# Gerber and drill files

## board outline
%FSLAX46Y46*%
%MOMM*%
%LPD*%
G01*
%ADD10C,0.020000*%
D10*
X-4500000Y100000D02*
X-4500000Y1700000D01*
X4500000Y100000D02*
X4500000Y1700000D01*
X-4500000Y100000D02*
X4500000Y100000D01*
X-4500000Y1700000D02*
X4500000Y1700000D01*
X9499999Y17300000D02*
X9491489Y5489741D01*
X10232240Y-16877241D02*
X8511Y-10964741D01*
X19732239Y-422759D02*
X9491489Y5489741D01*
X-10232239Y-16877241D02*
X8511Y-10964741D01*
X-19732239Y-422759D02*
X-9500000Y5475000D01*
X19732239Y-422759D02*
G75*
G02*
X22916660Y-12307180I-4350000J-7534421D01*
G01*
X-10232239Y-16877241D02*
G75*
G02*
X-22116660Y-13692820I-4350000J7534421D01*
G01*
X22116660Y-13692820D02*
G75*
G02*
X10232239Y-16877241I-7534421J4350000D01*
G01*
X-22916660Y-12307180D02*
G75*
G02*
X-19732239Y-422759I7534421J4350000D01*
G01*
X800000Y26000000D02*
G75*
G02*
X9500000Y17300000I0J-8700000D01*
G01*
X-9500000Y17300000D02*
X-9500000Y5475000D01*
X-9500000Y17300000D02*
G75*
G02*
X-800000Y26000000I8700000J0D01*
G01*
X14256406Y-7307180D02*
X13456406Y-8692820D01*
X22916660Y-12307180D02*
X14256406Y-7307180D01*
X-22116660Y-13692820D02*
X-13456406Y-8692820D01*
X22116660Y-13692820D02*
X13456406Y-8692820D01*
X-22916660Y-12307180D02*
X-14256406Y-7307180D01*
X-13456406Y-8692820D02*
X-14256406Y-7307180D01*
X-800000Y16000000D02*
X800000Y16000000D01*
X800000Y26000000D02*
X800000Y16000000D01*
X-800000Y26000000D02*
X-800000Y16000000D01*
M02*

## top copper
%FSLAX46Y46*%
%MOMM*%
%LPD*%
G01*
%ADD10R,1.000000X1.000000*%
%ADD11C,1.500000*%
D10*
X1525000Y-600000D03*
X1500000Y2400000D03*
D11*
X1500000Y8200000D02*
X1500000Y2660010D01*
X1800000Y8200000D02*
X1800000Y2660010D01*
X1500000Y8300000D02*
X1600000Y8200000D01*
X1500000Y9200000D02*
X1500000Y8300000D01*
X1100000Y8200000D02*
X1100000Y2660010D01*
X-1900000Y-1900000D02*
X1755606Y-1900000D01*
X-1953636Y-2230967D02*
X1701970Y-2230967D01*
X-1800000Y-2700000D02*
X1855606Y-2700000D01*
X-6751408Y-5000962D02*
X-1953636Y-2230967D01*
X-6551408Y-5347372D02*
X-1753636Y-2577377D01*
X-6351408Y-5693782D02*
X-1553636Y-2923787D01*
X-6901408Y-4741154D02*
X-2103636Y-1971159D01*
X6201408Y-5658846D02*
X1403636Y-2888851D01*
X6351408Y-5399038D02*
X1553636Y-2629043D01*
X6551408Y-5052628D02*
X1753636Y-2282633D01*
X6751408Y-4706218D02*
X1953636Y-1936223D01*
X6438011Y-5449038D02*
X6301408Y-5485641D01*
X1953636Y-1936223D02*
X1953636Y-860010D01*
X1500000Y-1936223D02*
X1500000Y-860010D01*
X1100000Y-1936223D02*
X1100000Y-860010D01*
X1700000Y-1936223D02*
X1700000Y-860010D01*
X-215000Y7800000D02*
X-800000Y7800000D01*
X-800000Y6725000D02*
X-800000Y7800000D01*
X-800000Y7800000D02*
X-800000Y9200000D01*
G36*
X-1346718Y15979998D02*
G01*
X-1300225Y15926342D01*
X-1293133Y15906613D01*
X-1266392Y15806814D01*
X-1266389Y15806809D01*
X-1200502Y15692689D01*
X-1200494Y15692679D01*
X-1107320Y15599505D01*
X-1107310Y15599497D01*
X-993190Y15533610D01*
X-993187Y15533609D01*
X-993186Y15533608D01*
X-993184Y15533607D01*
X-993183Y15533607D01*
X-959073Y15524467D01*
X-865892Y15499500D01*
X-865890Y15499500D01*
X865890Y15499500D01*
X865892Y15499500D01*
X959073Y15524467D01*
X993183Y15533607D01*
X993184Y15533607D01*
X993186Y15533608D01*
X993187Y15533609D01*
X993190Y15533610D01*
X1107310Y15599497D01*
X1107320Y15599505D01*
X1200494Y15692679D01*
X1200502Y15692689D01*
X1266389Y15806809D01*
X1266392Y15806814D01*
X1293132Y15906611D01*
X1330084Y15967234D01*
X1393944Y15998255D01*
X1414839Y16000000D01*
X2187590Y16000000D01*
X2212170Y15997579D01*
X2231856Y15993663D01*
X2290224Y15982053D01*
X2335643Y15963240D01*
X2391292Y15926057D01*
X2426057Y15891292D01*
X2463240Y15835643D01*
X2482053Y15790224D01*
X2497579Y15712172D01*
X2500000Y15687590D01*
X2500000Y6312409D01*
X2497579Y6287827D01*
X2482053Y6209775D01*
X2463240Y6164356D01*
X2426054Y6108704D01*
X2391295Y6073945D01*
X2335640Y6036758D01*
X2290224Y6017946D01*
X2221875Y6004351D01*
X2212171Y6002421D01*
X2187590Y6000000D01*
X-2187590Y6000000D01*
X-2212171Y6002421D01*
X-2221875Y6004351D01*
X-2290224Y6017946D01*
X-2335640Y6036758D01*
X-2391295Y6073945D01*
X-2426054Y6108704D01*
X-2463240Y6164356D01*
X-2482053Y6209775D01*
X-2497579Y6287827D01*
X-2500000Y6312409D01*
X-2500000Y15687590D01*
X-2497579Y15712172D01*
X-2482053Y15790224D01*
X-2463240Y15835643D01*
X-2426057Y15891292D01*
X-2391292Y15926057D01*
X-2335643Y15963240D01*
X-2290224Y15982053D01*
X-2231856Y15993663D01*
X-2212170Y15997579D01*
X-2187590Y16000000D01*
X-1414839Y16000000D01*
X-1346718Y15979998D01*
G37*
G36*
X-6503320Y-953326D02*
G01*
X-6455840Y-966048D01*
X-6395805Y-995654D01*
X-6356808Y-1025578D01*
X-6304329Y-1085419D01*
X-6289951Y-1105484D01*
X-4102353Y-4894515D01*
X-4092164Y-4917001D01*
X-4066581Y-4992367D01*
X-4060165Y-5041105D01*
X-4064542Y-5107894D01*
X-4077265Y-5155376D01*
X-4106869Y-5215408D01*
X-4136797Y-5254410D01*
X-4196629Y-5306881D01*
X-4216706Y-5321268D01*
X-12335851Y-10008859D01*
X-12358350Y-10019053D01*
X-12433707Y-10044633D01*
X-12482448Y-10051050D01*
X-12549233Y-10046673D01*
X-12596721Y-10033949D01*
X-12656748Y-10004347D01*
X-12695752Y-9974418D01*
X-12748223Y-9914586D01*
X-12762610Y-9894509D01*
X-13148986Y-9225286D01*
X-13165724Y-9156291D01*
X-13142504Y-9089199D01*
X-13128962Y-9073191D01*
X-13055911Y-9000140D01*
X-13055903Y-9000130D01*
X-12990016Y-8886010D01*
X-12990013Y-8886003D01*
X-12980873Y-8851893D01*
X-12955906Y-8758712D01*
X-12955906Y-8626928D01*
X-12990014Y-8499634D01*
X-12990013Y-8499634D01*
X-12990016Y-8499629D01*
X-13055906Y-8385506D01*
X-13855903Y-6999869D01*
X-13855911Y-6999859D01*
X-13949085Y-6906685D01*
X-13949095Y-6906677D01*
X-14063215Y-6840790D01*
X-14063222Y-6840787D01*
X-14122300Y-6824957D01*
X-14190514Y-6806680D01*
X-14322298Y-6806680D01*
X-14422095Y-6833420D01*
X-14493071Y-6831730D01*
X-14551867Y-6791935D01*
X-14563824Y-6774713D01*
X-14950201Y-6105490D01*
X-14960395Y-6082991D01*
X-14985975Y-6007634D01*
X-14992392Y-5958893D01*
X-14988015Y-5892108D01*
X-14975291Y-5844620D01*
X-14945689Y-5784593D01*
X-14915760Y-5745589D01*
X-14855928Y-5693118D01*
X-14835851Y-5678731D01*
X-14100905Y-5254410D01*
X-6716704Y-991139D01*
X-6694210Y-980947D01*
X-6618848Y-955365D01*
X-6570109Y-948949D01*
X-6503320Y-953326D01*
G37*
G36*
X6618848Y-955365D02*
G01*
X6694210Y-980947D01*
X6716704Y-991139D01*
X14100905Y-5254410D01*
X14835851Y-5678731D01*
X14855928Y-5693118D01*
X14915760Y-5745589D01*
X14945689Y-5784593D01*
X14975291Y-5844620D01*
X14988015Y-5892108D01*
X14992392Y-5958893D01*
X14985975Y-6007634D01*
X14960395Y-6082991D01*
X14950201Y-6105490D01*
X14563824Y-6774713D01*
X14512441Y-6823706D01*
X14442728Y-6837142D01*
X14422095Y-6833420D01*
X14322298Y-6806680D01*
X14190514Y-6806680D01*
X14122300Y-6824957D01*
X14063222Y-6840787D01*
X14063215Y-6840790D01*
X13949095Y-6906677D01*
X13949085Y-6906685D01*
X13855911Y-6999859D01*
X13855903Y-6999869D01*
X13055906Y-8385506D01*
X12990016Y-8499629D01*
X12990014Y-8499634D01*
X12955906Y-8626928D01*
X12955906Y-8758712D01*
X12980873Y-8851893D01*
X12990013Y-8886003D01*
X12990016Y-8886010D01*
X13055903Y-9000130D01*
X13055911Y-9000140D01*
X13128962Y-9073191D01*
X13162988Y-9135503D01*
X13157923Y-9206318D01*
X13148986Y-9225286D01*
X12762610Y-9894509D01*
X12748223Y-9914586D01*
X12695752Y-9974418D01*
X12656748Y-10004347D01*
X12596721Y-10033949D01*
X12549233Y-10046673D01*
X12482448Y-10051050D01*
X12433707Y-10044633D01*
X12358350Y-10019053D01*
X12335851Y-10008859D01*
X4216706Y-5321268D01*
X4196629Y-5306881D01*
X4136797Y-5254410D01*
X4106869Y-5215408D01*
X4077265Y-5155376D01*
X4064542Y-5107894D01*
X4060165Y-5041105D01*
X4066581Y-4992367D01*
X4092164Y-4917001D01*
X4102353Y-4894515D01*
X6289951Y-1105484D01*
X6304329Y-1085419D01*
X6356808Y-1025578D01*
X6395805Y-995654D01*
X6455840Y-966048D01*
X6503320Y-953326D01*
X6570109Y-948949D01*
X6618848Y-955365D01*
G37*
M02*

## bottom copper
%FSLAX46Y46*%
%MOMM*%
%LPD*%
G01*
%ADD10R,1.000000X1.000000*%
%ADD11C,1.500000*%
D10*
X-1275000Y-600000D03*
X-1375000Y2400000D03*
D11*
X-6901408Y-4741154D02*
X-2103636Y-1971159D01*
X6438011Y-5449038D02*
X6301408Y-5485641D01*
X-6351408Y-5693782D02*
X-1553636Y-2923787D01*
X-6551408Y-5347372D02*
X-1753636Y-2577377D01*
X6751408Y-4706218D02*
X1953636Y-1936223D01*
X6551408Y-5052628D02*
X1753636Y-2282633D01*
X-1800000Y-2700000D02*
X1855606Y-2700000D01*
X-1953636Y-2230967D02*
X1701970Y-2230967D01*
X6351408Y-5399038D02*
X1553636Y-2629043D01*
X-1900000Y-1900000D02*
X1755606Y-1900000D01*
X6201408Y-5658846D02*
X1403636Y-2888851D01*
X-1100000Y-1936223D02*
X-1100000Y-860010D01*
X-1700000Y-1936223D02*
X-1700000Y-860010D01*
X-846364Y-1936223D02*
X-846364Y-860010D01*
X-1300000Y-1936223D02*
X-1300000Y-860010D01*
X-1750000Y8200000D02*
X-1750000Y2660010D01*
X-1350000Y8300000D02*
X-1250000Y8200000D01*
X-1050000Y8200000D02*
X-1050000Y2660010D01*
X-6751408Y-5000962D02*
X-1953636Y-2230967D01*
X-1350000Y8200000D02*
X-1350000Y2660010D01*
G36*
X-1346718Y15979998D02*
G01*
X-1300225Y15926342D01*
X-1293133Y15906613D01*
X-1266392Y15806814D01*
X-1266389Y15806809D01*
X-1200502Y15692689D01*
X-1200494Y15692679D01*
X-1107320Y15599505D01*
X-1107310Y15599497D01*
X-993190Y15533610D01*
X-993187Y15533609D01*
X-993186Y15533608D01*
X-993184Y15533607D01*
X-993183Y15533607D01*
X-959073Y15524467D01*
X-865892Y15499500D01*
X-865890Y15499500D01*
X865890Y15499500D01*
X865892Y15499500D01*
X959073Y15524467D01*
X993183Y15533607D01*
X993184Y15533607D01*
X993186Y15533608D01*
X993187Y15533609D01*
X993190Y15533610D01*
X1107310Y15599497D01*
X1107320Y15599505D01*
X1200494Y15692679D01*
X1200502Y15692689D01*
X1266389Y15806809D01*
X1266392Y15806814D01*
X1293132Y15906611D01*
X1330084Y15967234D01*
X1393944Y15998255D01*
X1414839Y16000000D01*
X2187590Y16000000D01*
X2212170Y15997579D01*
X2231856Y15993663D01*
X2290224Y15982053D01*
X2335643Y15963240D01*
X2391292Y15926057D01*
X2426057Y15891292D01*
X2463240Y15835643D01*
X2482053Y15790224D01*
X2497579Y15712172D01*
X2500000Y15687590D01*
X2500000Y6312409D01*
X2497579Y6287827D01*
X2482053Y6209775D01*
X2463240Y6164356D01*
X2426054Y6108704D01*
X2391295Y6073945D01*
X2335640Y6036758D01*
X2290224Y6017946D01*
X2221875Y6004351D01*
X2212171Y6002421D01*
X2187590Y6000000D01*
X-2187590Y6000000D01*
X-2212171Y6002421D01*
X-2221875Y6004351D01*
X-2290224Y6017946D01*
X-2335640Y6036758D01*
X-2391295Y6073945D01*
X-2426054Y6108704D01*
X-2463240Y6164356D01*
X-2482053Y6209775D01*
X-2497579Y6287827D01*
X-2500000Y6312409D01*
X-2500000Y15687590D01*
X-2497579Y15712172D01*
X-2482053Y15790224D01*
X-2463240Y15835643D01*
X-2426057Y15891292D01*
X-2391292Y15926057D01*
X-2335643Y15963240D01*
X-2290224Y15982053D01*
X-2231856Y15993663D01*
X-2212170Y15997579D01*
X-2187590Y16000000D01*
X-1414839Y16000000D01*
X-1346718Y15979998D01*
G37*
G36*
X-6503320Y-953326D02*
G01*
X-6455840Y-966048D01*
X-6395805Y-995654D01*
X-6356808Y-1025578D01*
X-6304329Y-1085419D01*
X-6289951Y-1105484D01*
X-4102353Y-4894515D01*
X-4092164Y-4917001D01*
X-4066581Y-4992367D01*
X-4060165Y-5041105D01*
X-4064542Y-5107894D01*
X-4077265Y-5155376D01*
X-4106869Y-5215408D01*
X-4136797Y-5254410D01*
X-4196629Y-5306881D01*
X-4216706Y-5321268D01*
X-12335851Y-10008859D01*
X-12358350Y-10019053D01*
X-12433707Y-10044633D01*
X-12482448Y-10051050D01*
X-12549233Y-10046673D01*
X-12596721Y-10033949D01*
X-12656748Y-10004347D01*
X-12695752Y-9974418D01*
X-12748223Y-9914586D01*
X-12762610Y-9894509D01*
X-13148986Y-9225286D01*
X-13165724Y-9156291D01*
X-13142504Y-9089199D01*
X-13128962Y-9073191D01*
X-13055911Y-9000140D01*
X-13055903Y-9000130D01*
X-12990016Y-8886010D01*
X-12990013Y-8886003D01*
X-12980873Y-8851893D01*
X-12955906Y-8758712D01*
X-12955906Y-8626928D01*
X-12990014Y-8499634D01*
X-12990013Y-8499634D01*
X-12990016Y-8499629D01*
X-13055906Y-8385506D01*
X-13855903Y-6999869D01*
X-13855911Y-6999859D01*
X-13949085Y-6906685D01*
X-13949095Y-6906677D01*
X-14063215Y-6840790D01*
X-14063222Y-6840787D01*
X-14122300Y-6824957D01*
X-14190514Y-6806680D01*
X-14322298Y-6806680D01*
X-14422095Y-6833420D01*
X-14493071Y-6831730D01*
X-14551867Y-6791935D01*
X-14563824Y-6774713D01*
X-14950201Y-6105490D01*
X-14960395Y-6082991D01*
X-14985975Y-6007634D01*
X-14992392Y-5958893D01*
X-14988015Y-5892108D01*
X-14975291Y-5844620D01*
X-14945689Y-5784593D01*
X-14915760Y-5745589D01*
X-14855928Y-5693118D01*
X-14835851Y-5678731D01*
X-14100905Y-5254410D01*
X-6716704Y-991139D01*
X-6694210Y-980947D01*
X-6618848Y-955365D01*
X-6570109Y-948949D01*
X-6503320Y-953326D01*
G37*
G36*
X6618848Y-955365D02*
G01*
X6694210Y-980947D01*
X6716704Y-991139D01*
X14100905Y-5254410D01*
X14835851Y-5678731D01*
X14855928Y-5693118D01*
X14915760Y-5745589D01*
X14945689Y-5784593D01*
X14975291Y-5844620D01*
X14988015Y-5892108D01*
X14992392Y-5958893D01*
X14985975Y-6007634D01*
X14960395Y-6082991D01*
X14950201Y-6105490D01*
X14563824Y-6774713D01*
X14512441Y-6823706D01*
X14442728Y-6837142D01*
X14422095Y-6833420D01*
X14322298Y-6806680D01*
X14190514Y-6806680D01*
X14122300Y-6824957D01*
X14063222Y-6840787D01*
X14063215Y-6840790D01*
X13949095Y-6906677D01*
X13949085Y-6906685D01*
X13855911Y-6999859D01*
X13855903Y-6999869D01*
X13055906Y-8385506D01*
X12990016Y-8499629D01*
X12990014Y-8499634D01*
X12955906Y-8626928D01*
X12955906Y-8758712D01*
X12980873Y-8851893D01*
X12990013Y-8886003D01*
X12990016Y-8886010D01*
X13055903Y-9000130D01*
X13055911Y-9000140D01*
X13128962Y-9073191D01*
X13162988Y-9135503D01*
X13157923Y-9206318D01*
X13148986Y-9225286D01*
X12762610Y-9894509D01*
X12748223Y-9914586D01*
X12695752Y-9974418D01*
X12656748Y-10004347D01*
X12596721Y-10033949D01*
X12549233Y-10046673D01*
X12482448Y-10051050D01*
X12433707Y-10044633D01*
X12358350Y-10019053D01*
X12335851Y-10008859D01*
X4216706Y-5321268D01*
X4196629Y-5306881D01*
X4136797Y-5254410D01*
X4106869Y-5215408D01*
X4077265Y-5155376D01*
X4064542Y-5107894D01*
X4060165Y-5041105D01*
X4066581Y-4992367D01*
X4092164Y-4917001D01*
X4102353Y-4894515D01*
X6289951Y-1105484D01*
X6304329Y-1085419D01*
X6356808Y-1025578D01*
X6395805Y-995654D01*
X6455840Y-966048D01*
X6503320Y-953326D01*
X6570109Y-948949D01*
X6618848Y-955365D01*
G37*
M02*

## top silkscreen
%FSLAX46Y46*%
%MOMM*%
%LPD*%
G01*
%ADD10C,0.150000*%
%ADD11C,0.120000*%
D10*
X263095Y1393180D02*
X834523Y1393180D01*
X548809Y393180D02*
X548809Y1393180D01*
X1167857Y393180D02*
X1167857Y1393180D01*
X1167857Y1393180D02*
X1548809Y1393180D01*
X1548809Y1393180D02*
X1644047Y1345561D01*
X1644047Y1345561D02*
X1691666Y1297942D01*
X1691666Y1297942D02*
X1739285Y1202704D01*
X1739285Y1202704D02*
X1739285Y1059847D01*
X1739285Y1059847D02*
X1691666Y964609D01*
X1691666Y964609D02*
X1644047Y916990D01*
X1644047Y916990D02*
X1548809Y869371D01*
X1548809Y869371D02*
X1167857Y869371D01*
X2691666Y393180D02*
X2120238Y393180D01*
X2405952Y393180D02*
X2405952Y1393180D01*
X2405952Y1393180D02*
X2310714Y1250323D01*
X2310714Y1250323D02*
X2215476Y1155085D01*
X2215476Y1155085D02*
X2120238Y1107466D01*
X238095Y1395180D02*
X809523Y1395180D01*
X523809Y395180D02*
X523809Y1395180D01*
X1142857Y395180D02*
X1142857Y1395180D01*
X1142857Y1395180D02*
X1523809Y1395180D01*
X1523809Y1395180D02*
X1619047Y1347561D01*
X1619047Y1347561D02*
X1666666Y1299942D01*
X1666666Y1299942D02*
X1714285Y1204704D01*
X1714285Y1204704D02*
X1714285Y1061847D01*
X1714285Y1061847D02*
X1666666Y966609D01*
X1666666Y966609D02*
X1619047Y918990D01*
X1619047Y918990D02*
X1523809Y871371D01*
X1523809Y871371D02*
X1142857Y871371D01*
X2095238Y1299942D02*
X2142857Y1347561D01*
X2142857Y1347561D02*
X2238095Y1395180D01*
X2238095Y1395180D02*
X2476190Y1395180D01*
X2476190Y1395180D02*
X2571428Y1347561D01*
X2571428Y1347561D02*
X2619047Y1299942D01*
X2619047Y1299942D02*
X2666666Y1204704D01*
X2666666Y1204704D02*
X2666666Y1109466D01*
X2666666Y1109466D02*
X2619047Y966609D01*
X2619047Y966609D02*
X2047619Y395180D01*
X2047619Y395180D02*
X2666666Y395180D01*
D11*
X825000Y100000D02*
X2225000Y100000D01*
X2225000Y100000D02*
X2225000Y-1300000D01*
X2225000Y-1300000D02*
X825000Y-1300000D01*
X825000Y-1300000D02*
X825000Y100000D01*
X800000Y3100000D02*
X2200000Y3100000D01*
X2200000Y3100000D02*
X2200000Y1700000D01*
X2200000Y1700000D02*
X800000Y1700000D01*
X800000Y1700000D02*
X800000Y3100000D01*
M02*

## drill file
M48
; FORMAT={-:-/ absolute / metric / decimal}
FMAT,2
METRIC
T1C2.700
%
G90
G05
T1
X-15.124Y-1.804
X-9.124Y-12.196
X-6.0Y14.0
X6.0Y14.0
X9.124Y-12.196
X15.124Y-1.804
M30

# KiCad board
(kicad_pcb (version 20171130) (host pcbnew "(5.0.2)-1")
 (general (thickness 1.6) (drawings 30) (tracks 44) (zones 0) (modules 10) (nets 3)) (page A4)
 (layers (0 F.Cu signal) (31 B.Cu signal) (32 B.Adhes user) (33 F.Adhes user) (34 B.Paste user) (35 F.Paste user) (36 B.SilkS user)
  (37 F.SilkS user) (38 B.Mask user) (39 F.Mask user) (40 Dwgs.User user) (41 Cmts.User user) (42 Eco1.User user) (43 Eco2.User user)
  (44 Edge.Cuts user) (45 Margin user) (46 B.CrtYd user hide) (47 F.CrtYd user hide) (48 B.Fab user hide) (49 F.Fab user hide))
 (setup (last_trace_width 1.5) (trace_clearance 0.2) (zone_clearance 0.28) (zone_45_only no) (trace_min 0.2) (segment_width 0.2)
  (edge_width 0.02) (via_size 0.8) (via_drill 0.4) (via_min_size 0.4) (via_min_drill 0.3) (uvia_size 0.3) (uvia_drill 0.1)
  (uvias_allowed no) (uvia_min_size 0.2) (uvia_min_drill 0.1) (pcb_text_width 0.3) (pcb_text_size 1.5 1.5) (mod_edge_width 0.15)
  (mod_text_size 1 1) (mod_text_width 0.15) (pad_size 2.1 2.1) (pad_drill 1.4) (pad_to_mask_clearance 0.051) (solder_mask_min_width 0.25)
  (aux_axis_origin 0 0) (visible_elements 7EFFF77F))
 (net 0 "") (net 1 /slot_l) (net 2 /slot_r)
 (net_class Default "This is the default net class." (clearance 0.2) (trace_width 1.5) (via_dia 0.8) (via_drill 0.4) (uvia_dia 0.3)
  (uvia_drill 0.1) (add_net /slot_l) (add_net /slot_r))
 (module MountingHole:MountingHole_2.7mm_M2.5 (layer F.Cu) (at 15.124356 1.803848 240)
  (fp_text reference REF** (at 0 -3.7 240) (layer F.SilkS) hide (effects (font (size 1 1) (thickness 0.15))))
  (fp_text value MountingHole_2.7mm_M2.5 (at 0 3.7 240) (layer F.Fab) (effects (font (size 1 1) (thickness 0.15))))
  (pad 1 np_thru_hole circle (at 0 0 240) (size 2.7 2.7) (drill 2.7) (layers *.Cu *.Mask)))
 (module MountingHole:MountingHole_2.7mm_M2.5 (layer F.Cu) (at -9.124356 12.196152 120)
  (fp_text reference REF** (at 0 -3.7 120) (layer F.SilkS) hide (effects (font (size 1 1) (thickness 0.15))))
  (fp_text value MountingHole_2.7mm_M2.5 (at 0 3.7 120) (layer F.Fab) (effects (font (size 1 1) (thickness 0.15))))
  (pad 1 np_thru_hole circle (at 0 0 120) (size 2.7 2.7) (drill 2.7) (layers *.Cu *.Mask)))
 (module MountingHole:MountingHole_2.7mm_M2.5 (layer F.Cu) (at 9.124356 12.196152 240)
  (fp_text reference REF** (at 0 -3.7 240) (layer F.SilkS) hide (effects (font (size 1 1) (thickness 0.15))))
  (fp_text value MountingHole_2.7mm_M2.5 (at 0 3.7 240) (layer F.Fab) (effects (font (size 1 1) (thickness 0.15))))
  (pad 1 np_thru_hole circle (at 0 0 240) (size 2.7 2.7) (drill 2.7) (layers *.Cu *.Mask)))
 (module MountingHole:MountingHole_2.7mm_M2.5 (layer F.Cu) (at -15.124356 1.803848 120)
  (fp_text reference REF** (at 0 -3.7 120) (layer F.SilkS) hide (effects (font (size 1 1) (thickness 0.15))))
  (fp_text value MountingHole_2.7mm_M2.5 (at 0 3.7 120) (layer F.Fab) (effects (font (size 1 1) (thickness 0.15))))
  (pad 1 np_thru_hole circle (at 0 0 120) (size 2.7 2.7) (drill 2.7) (layers *.Cu *.Mask)))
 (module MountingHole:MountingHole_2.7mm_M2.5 (layer F.Cu) (at 6 -14)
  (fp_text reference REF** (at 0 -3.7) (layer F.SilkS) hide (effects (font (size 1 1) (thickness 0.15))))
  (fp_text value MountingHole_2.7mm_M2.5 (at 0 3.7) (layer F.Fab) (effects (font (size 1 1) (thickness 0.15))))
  (pad 1 np_thru_hole circle (at 0 0) (size 2.7 2.7) (drill 2.7) (layers *.Cu *.Mask)))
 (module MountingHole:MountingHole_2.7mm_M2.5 (layer F.Cu) (at -6 -14)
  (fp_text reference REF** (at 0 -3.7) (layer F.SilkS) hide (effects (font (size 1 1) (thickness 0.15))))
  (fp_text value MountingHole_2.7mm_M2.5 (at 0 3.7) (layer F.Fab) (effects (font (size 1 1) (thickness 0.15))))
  (pad 1 np_thru_hole circle (at 0 0) (size 2.7 2.7) (drill 2.7) (layers *.Cu *.Mask)))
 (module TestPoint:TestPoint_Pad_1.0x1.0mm (layer F.Cu) (at 1.525 0.6)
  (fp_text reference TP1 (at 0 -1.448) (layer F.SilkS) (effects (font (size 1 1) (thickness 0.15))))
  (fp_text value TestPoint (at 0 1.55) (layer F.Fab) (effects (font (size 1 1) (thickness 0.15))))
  (fp_line (start -0.7 -0.7) (end 0.7 -0.7) (layer F.SilkS) (width 0.12))
  (fp_line (start 0.7 -0.7) (end 0.7 0.7) (layer F.SilkS) (width 0.12))
  (fp_line (start 0.7 0.7) (end -0.7 0.7) (layer F.SilkS) (width 0.12))
  (fp_line (start -0.7 0.7) (end -0.7 -0.7) (layer F.SilkS) (width 0.12))
  (pad 1 smd rect (at 0 0) (size 1 1) (layers F.Cu F.Mask) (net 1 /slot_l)))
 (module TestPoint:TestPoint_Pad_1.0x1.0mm (layer F.Cu) (at 1.5 -2.4)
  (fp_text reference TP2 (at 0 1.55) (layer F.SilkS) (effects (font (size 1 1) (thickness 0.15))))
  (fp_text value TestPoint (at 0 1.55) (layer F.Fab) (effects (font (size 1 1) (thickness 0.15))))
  (fp_line (start -0.7 -0.7) (end 0.7 -0.7) (layer F.SilkS) (width 0.12))
  (fp_line (start 0.7 -0.7) (end 0.7 0.7) (layer F.SilkS) (width 0.12))
  (fp_line (start 0.7 0.7) (end -0.7 0.7) (layer F.SilkS) (width 0.12))
  (fp_line (start -0.7 0.7) (end -0.7 -0.7) (layer F.SilkS) (width 0.12))
  (pad 1 smd rect (at 0 0) (size 1 1) (layers F.Cu F.Mask) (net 1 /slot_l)))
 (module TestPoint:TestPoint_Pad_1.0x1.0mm (layer B.Cu) (at -1.275 0.6)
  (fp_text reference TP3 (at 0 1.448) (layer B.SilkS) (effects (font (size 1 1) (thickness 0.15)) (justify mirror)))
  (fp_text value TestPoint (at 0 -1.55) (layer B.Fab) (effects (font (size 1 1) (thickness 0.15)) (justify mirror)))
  (pad 1 smd rect (at 0 0) (size 1 1) (layers B.Cu B.Mask) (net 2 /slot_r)))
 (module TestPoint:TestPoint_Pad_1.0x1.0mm (layer B.Cu) (at -1.375 -2.4)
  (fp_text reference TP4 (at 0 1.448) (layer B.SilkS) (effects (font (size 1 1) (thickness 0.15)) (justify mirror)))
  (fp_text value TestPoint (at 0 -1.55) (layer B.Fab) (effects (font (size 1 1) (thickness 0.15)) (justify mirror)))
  (pad 1 smd rect (at 0 0) (size 1 1) (layers B.Cu B.Mask) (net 2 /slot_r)))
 (gr_line (start -4.5 -0.1) (end -4.5 -1.7) (layer Edge.Cuts) (width 0.02))
 (gr_line (start 4.5 -0.1) (end 4.5 -1.7) (layer Edge.Cuts) (width 0.02))
 (gr_line (start -4.5 -0.1) (end 4.5 -0.1) (layer Edge.Cuts) (width 0.02))
 (gr_line (start -4.5 -1.7) (end 4.5 -1.7) (layer Edge.Cuts) (width 0.02))
 (gr_line (start 9.499999 -17.3) (end 9.491489 -5.489741) (layer Edge.Cuts) (width 0.02))
 (gr_line (start 10.23224 16.877241) (end 0.008511 10.964741) (layer Edge.Cuts) (width 0.02))
 (gr_line (start 19.732239 0.422759) (end 9.491489 -5.489741) (layer Edge.Cuts) (width 0.02))
 (gr_line (start -10.232239 16.877241) (end 0.008511 10.964741) (layer Edge.Cuts) (width 0.02))
 (gr_line (start -19.732239 0.422759) (end -9.5 -5.475) (layer Edge.Cuts) (width 0.02))
 (gr_arc (start 15.382239 7.95718) (end 22.91666 12.30718) (angle -90) (layer Edge.Cuts) (width 0.02))
 (gr_arc (start -14.582239 9.34282) (end -22.11666 13.69282) (angle -90) (layer Edge.Cuts) (width 0.02))
 (gr_arc (start 14.582239 9.34282) (end 10.232239 16.877241) (angle -90) (layer Edge.Cuts) (width 0.02))
 (gr_arc (start -15.382239 7.95718) (end -19.732239 0.422759) (angle -90) (layer Edge.Cuts) (width 0.02))
 (gr_arc (start 0.8 -17.3) (end 9.5 -17.3) (angle -90) (layer Edge.Cuts) (width 0.02))
 (gr_line (start -9.5 -17.3) (end -9.5 -5.475) (layer Edge.Cuts) (width 0.02))
 (gr_arc (start -0.8 -17.3) (end -0.8 -26) (angle -90) (layer Edge.Cuts) (width 0.02))
 (gr_line (start 14.256406 7.30718) (end 13.456406 8.69282) (layer Edge.Cuts) (width 0.02))
 (gr_line (start 22.91666 12.30718) (end 14.256406 7.30718) (layer Edge.Cuts) (width 0.02))
 (gr_line (start -22.11666 13.69282) (end -13.456406 8.69282) (layer Edge.Cuts) (width 0.02))
 (gr_line (start 22.11666 13.69282) (end 13.456406 8.69282) (layer Edge.Cuts) (width 0.02))
 (gr_line (start -22.91666 12.30718) (end -14.256406 7.30718) (layer Edge.Cuts) (width 0.02))
 (gr_line (start -13.456406 8.69282) (end -14.256406 7.30718) (layer Edge.Cuts) (width 0.02))
 (gr_line (start -0.8 -16) (end 0.8 -16) (layer Edge.Cuts) (width 0.02))
 (gr_line (start 0.8 -26) (end 0.8 -16) (layer Edge.Cuts) (width 0.02))
 (gr_line (start -0.8 -26) (end -0.8 -16) (layer Edge.Cuts) (width 0.02))
 (segment (start 1.5 -8.2) (end 1.5 -2.66001) (width 1.5) (layer F.Cu) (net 1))
 (segment (start 1.8 -8.2) (end 1.8 -2.66001) (width 1.5) (layer F.Cu) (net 1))
 (segment (start 1.5 -8.3) (end 1.6 -8.2) (width 1.5) (layer F.Cu) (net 1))
 (segment (start 1.5 -9.2) (end 1.5 -8.3) (width 1.5) (layer F.Cu) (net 1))
 (segment (start 1.1 -8.2) (end 1.1 -2.66001) (width 1.5) (layer F.Cu) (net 1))
 (segment (start -1.9 1.9) (end 1.755606 1.9) (width 1.5) (layer F.Cu) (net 1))
 (segment (start -1.953636 2.230967) (end 1.70197 2.230967) (width 1.5) (layer F.Cu) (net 1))
 (segment (start -1.8 2.7) (end 1.855606 2.7) (width 1.5) (layer F.Cu) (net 1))
 (segment (start -6.751408 5.000962) (end -1.953636 2.230967) (width 1.5) (layer F.Cu) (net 1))
 (segment (start -6.551408 5.347372) (end -1.753636 2.577377) (width 1.5) (layer F.Cu) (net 1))
 (segment (start -6.351408 5.693782) (end -1.553636 2.923787) (width 1.5) (layer F.Cu) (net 1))
 (segment (start -6.901408 4.741154) (end -2.103636 1.971159) (width 1.5) (layer F.Cu) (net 1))
 (segment (start 6.201408 5.658846) (end 1.403636 2.888851) (width 1.5) (layer F.Cu) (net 1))
 (segment (start 6.351408 5.399038) (end 1.553636 2.629043) (width 1.5) (layer F.Cu) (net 1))
 (segment (start 6.551408 5.052628) (end 1.753636 2.282633) (width 1.5) (layer F.Cu) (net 1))
 (segment (start 6.751408 4.706218) (end 1.953636 1.936223) (width 1.5) (layer F.Cu) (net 1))
 (segment (start 6.438011 5.449038) (end 6.301408 5.485641) (width 1.5) (layer F.Cu) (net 1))
 (segment (start 1.953636 1.936223) (end 1.953636 0.86001) (width 1.5) (layer F.Cu) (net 1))
 (segment (start 1.5 1.936223) (end 1.5 0.86001) (width 1.5) (layer F.Cu) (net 1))
 (segment (start 1.1 1.936223) (end 1.1 0.86001) (width 1.5) (layer F.Cu) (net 1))
 (segment (start 1.7 1.936223) (end 1.7 0.86001) (width 1.5) (layer F.Cu) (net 1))
 (segment (start -6.901408 4.741154) (end -2.103636 1.971159) (width 1.5) (layer B.Cu) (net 2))
 (segment (start 6.438011 5.449038) (end 6.301408 5.485641) (width 1.5) (layer B.Cu) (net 2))
 (segment (start -6.351408 5.693782) (end -1.553636 2.923787) (width 1.5) (layer B.Cu) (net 2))
 (segment (start -6.551408 5.347372) (end -1.753636 2.577377) (width 1.5) (layer B.Cu) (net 2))
 (segment (start 6.751408 4.706218) (end 1.953636 1.936223) (width 1.5) (layer B.Cu) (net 2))
 (segment (start 6.551408 5.052628) (end 1.753636 2.282633) (width 1.5) (layer B.Cu) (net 2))
 (segment (start -1.8 2.7) (end 1.855606 2.7) (width 1.5) (layer B.Cu) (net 2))
 (segment (start -1.953636 2.230967) (end 1.70197 2.230967) (width 1.5) (layer B.Cu) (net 2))
 (segment (start 6.351408 5.399038) (end 1.553636 2.629043) (width 1.5) (layer B.Cu) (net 2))
 (segment (start -1.9 1.9) (end 1.755606 1.9) (width 1.5) (layer B.Cu) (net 2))
 (segment (start 6.201408 5.658846) (end 1.403636 2.888851) (width 1.5) (layer B.Cu) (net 2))
 (segment (start -1.1 1.936223) (end -1.1 0.86001) (width 1.5) (layer B.Cu) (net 2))
 (segment (start -1.7 1.936223) (end -1.7 0.86001) (width 1.5) (layer B.Cu) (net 2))
 (segment (start -0.846364 1.936223) (end -0.846364 0.86001) (width 1.5) (layer B.Cu) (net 2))
 (segment (start -1.3 1.936223) (end -1.3 0.86001) (width 1.5) (layer B.Cu) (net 2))
 (segment (start -1.75 -8.2) (end -1.75 -2.66001) (width 1.5) (layer B.Cu) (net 2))
 (segment (start -1.35 -8.3) (end -1.25 -8.2) (width 1.5) (layer B.Cu) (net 2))
 (segment (start -1.05 -8.2) (end -1.05 -2.66001) (width 1.5) (layer B.Cu) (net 2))
 (segment (start -6.751408 5.000962) (end -1.953636 2.230967) (width 1.5) (layer B.Cu) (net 2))
 (segment (start -1.35 -8.2) (end -1.35 -2.66001) (width 1.5) (layer B.Cu) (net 2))
 (segment (start -0.215 -7.8) (end -0.8 -7.8) (width 1.5) (layer F.Cu) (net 1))
 (segment (start -0.8 -6.725) (end -0.8 -7.8) (width 1.5) (layer F.Cu) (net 1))
 (segment (start -0.8 -7.8) (end -0.8 -9.2) (width 1.5) (layer F.Cu) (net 1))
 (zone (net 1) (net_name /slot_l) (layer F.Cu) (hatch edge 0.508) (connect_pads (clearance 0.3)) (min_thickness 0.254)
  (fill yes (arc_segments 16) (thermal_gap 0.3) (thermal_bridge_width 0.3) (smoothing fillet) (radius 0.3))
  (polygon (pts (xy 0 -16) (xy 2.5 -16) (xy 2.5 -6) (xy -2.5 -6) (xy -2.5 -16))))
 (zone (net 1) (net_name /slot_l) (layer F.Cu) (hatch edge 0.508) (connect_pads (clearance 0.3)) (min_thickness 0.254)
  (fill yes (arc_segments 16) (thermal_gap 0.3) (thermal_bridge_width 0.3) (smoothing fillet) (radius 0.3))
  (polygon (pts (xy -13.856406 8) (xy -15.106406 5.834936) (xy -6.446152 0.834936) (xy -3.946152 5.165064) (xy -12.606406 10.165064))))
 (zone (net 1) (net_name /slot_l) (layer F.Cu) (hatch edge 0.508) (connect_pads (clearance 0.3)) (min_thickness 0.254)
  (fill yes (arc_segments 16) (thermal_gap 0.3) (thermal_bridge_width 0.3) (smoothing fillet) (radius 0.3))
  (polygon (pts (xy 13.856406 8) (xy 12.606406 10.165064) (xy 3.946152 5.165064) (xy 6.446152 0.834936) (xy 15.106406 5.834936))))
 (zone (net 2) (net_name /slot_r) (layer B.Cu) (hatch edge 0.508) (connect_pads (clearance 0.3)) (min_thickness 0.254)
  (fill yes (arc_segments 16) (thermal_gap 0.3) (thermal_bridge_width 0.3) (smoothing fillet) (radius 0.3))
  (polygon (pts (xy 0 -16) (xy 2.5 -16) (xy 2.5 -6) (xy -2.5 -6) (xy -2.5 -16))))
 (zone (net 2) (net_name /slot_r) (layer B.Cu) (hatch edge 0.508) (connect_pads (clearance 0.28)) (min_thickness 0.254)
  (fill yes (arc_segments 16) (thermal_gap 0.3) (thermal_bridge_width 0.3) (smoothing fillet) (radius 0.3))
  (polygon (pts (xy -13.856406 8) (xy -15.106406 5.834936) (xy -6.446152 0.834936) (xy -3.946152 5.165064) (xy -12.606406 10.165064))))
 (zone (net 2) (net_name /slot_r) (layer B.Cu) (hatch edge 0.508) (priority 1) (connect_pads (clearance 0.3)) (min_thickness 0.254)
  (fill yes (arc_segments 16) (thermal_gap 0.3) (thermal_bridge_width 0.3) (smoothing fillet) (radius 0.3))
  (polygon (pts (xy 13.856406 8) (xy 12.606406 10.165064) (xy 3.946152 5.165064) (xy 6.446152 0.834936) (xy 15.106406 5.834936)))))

